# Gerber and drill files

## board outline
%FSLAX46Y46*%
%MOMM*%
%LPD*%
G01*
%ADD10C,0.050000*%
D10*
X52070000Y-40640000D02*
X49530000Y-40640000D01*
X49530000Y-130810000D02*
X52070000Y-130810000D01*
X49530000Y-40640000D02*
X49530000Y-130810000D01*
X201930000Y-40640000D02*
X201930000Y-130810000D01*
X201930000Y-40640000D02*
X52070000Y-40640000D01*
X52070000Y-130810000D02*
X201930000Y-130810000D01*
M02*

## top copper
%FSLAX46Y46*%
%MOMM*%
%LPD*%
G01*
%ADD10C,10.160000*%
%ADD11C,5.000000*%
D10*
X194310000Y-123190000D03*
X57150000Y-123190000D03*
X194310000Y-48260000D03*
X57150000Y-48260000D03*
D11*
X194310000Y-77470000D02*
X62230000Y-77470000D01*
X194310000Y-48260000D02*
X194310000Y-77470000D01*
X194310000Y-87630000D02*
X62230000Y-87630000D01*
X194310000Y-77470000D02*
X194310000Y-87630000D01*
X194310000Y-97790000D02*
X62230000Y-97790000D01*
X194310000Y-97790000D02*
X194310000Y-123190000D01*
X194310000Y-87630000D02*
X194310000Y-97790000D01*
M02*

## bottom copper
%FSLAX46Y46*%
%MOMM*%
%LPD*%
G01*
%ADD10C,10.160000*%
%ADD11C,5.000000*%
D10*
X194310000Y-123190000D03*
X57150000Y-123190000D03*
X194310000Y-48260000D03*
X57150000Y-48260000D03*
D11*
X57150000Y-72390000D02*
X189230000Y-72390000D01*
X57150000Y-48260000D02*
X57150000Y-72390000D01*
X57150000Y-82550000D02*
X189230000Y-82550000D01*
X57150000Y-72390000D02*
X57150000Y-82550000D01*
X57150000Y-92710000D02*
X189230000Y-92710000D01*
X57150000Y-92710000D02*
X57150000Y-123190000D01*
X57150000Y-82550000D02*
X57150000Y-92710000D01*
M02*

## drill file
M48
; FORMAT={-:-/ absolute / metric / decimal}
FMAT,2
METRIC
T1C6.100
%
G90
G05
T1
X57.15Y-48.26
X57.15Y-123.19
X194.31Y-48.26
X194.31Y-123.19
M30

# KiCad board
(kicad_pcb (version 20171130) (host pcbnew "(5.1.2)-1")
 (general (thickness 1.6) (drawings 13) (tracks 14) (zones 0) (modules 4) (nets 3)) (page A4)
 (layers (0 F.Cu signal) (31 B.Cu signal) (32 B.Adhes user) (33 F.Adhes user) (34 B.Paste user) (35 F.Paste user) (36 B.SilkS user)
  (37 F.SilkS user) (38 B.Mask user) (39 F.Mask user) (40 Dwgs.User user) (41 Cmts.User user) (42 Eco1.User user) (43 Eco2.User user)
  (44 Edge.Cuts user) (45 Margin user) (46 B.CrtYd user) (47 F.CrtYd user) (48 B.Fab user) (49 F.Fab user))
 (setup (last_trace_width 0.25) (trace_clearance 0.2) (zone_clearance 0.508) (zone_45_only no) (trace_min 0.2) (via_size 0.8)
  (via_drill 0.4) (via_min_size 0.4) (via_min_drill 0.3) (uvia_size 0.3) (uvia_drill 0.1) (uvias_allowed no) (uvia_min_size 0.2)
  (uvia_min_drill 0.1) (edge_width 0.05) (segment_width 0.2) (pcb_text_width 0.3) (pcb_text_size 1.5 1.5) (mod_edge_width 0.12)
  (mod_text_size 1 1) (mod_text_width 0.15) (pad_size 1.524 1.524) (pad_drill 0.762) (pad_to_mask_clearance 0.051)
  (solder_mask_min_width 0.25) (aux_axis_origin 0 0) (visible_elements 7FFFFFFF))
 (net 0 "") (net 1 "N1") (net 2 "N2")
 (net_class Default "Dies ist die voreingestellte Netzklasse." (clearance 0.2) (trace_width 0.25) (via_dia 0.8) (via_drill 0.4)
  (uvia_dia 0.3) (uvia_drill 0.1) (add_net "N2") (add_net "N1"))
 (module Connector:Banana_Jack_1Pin (layer F.Cu) (at 194.31 123.19)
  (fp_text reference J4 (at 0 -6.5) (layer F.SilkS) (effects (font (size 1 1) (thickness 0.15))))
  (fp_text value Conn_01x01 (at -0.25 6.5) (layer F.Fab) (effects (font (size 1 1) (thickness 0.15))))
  (pad 1 thru_hole circle (at 0 0) (size 10.16 10.16) (drill 6.1) (layers *.Cu *.Mask) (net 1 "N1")))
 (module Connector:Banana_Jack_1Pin (layer F.Cu) (at 57.15 123.19)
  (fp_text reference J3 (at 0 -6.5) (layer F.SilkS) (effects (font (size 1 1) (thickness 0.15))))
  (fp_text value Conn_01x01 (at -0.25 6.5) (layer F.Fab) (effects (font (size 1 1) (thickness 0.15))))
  (pad 1 thru_hole circle (at 0 0) (size 10.16 10.16) (drill 6.1) (layers *.Cu *.Mask) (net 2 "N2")))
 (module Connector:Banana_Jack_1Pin (layer F.Cu) (at 194.31 48.26 180)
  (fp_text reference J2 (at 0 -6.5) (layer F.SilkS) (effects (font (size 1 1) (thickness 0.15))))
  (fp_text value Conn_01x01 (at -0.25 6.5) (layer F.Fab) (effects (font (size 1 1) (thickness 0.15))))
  (pad 1 thru_hole circle (at 0 0 180) (size 10.16 10.16) (drill 6.1) (layers *.Cu *.Mask) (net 1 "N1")))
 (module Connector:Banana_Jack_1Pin (layer F.Cu) (at 57.15 48.26 180)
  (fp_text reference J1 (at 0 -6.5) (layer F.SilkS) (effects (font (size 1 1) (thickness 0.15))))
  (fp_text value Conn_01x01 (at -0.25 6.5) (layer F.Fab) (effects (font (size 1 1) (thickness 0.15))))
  (pad 1 thru_hole circle (at 0 0 180) (size 10.16 10.16) (drill 6.1) (layers *.Cu *.Mask) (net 2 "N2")))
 (gr_line (start 52.07 40.64) (end 49.53 40.64) (layer Edge.Cuts) (width 0.05))
 (gr_line (start 49.53 130.81) (end 52.07 130.81) (layer Edge.Cuts) (width 0.05))
 (gr_line (start 49.53 40.64) (end 49.53 130.81) (layer Edge.Cuts) (width 0.05))
 (gr_line (start 201.93 40.64) (end 201.93 130.81) (layer Edge.Cuts) (width 0.05))
 (gr_line (start 201.93 40.64) (end 52.07 40.64) (layer Edge.Cuts) (width 0.05))
 (gr_line (start 52.07 130.81) (end 201.93 130.81) (layer Edge.Cuts) (width 0.05))
 (segment (start 57.15 72.39) (end 189.23 72.39) (width 5) (layer B.Cu) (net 2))
 (segment (start 57.15 48.26) (end 57.15 72.39) (width 5) (layer B.Cu) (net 2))
 (segment (start 57.15 82.55) (end 189.23 82.55) (width 5) (layer B.Cu) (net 2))
 (segment (start 57.15 72.39) (end 57.15 82.55) (width 5) (layer B.Cu) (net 2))
 (segment (start 57.15 92.71) (end 189.23 92.71) (width 5) (layer B.Cu) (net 2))
 (segment (start 57.15 92.71) (end 57.15 123.19) (width 5) (layer B.Cu) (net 2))
 (segment (start 57.15 82.55) (end 57.15 92.71) (width 5) (layer B.Cu) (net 2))
 (segment (start 194.31 77.47) (end 62.23 77.47) (width 5) (layer F.Cu) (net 1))
 (segment (start 194.31 48.26) (end 194.31 77.47) (width 5) (layer F.Cu) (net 1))
 (segment (start 194.31 87.63) (end 62.23 87.63) (width 5) (layer F.Cu) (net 1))
 (segment (start 194.31 77.47) (end 194.31 87.63) (width 5) (layer F.Cu) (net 1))
 (segment (start 194.31 97.79) (end 62.23 97.79) (width 5) (layer F.Cu) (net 1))
 (segment (start 194.31 97.79) (end 194.31 123.19) (width 5) (layer F.Cu) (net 1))
 (segment (start 194.31 87.63) (end 194.31 97.79) (width 5) (layer F.Cu) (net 1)))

